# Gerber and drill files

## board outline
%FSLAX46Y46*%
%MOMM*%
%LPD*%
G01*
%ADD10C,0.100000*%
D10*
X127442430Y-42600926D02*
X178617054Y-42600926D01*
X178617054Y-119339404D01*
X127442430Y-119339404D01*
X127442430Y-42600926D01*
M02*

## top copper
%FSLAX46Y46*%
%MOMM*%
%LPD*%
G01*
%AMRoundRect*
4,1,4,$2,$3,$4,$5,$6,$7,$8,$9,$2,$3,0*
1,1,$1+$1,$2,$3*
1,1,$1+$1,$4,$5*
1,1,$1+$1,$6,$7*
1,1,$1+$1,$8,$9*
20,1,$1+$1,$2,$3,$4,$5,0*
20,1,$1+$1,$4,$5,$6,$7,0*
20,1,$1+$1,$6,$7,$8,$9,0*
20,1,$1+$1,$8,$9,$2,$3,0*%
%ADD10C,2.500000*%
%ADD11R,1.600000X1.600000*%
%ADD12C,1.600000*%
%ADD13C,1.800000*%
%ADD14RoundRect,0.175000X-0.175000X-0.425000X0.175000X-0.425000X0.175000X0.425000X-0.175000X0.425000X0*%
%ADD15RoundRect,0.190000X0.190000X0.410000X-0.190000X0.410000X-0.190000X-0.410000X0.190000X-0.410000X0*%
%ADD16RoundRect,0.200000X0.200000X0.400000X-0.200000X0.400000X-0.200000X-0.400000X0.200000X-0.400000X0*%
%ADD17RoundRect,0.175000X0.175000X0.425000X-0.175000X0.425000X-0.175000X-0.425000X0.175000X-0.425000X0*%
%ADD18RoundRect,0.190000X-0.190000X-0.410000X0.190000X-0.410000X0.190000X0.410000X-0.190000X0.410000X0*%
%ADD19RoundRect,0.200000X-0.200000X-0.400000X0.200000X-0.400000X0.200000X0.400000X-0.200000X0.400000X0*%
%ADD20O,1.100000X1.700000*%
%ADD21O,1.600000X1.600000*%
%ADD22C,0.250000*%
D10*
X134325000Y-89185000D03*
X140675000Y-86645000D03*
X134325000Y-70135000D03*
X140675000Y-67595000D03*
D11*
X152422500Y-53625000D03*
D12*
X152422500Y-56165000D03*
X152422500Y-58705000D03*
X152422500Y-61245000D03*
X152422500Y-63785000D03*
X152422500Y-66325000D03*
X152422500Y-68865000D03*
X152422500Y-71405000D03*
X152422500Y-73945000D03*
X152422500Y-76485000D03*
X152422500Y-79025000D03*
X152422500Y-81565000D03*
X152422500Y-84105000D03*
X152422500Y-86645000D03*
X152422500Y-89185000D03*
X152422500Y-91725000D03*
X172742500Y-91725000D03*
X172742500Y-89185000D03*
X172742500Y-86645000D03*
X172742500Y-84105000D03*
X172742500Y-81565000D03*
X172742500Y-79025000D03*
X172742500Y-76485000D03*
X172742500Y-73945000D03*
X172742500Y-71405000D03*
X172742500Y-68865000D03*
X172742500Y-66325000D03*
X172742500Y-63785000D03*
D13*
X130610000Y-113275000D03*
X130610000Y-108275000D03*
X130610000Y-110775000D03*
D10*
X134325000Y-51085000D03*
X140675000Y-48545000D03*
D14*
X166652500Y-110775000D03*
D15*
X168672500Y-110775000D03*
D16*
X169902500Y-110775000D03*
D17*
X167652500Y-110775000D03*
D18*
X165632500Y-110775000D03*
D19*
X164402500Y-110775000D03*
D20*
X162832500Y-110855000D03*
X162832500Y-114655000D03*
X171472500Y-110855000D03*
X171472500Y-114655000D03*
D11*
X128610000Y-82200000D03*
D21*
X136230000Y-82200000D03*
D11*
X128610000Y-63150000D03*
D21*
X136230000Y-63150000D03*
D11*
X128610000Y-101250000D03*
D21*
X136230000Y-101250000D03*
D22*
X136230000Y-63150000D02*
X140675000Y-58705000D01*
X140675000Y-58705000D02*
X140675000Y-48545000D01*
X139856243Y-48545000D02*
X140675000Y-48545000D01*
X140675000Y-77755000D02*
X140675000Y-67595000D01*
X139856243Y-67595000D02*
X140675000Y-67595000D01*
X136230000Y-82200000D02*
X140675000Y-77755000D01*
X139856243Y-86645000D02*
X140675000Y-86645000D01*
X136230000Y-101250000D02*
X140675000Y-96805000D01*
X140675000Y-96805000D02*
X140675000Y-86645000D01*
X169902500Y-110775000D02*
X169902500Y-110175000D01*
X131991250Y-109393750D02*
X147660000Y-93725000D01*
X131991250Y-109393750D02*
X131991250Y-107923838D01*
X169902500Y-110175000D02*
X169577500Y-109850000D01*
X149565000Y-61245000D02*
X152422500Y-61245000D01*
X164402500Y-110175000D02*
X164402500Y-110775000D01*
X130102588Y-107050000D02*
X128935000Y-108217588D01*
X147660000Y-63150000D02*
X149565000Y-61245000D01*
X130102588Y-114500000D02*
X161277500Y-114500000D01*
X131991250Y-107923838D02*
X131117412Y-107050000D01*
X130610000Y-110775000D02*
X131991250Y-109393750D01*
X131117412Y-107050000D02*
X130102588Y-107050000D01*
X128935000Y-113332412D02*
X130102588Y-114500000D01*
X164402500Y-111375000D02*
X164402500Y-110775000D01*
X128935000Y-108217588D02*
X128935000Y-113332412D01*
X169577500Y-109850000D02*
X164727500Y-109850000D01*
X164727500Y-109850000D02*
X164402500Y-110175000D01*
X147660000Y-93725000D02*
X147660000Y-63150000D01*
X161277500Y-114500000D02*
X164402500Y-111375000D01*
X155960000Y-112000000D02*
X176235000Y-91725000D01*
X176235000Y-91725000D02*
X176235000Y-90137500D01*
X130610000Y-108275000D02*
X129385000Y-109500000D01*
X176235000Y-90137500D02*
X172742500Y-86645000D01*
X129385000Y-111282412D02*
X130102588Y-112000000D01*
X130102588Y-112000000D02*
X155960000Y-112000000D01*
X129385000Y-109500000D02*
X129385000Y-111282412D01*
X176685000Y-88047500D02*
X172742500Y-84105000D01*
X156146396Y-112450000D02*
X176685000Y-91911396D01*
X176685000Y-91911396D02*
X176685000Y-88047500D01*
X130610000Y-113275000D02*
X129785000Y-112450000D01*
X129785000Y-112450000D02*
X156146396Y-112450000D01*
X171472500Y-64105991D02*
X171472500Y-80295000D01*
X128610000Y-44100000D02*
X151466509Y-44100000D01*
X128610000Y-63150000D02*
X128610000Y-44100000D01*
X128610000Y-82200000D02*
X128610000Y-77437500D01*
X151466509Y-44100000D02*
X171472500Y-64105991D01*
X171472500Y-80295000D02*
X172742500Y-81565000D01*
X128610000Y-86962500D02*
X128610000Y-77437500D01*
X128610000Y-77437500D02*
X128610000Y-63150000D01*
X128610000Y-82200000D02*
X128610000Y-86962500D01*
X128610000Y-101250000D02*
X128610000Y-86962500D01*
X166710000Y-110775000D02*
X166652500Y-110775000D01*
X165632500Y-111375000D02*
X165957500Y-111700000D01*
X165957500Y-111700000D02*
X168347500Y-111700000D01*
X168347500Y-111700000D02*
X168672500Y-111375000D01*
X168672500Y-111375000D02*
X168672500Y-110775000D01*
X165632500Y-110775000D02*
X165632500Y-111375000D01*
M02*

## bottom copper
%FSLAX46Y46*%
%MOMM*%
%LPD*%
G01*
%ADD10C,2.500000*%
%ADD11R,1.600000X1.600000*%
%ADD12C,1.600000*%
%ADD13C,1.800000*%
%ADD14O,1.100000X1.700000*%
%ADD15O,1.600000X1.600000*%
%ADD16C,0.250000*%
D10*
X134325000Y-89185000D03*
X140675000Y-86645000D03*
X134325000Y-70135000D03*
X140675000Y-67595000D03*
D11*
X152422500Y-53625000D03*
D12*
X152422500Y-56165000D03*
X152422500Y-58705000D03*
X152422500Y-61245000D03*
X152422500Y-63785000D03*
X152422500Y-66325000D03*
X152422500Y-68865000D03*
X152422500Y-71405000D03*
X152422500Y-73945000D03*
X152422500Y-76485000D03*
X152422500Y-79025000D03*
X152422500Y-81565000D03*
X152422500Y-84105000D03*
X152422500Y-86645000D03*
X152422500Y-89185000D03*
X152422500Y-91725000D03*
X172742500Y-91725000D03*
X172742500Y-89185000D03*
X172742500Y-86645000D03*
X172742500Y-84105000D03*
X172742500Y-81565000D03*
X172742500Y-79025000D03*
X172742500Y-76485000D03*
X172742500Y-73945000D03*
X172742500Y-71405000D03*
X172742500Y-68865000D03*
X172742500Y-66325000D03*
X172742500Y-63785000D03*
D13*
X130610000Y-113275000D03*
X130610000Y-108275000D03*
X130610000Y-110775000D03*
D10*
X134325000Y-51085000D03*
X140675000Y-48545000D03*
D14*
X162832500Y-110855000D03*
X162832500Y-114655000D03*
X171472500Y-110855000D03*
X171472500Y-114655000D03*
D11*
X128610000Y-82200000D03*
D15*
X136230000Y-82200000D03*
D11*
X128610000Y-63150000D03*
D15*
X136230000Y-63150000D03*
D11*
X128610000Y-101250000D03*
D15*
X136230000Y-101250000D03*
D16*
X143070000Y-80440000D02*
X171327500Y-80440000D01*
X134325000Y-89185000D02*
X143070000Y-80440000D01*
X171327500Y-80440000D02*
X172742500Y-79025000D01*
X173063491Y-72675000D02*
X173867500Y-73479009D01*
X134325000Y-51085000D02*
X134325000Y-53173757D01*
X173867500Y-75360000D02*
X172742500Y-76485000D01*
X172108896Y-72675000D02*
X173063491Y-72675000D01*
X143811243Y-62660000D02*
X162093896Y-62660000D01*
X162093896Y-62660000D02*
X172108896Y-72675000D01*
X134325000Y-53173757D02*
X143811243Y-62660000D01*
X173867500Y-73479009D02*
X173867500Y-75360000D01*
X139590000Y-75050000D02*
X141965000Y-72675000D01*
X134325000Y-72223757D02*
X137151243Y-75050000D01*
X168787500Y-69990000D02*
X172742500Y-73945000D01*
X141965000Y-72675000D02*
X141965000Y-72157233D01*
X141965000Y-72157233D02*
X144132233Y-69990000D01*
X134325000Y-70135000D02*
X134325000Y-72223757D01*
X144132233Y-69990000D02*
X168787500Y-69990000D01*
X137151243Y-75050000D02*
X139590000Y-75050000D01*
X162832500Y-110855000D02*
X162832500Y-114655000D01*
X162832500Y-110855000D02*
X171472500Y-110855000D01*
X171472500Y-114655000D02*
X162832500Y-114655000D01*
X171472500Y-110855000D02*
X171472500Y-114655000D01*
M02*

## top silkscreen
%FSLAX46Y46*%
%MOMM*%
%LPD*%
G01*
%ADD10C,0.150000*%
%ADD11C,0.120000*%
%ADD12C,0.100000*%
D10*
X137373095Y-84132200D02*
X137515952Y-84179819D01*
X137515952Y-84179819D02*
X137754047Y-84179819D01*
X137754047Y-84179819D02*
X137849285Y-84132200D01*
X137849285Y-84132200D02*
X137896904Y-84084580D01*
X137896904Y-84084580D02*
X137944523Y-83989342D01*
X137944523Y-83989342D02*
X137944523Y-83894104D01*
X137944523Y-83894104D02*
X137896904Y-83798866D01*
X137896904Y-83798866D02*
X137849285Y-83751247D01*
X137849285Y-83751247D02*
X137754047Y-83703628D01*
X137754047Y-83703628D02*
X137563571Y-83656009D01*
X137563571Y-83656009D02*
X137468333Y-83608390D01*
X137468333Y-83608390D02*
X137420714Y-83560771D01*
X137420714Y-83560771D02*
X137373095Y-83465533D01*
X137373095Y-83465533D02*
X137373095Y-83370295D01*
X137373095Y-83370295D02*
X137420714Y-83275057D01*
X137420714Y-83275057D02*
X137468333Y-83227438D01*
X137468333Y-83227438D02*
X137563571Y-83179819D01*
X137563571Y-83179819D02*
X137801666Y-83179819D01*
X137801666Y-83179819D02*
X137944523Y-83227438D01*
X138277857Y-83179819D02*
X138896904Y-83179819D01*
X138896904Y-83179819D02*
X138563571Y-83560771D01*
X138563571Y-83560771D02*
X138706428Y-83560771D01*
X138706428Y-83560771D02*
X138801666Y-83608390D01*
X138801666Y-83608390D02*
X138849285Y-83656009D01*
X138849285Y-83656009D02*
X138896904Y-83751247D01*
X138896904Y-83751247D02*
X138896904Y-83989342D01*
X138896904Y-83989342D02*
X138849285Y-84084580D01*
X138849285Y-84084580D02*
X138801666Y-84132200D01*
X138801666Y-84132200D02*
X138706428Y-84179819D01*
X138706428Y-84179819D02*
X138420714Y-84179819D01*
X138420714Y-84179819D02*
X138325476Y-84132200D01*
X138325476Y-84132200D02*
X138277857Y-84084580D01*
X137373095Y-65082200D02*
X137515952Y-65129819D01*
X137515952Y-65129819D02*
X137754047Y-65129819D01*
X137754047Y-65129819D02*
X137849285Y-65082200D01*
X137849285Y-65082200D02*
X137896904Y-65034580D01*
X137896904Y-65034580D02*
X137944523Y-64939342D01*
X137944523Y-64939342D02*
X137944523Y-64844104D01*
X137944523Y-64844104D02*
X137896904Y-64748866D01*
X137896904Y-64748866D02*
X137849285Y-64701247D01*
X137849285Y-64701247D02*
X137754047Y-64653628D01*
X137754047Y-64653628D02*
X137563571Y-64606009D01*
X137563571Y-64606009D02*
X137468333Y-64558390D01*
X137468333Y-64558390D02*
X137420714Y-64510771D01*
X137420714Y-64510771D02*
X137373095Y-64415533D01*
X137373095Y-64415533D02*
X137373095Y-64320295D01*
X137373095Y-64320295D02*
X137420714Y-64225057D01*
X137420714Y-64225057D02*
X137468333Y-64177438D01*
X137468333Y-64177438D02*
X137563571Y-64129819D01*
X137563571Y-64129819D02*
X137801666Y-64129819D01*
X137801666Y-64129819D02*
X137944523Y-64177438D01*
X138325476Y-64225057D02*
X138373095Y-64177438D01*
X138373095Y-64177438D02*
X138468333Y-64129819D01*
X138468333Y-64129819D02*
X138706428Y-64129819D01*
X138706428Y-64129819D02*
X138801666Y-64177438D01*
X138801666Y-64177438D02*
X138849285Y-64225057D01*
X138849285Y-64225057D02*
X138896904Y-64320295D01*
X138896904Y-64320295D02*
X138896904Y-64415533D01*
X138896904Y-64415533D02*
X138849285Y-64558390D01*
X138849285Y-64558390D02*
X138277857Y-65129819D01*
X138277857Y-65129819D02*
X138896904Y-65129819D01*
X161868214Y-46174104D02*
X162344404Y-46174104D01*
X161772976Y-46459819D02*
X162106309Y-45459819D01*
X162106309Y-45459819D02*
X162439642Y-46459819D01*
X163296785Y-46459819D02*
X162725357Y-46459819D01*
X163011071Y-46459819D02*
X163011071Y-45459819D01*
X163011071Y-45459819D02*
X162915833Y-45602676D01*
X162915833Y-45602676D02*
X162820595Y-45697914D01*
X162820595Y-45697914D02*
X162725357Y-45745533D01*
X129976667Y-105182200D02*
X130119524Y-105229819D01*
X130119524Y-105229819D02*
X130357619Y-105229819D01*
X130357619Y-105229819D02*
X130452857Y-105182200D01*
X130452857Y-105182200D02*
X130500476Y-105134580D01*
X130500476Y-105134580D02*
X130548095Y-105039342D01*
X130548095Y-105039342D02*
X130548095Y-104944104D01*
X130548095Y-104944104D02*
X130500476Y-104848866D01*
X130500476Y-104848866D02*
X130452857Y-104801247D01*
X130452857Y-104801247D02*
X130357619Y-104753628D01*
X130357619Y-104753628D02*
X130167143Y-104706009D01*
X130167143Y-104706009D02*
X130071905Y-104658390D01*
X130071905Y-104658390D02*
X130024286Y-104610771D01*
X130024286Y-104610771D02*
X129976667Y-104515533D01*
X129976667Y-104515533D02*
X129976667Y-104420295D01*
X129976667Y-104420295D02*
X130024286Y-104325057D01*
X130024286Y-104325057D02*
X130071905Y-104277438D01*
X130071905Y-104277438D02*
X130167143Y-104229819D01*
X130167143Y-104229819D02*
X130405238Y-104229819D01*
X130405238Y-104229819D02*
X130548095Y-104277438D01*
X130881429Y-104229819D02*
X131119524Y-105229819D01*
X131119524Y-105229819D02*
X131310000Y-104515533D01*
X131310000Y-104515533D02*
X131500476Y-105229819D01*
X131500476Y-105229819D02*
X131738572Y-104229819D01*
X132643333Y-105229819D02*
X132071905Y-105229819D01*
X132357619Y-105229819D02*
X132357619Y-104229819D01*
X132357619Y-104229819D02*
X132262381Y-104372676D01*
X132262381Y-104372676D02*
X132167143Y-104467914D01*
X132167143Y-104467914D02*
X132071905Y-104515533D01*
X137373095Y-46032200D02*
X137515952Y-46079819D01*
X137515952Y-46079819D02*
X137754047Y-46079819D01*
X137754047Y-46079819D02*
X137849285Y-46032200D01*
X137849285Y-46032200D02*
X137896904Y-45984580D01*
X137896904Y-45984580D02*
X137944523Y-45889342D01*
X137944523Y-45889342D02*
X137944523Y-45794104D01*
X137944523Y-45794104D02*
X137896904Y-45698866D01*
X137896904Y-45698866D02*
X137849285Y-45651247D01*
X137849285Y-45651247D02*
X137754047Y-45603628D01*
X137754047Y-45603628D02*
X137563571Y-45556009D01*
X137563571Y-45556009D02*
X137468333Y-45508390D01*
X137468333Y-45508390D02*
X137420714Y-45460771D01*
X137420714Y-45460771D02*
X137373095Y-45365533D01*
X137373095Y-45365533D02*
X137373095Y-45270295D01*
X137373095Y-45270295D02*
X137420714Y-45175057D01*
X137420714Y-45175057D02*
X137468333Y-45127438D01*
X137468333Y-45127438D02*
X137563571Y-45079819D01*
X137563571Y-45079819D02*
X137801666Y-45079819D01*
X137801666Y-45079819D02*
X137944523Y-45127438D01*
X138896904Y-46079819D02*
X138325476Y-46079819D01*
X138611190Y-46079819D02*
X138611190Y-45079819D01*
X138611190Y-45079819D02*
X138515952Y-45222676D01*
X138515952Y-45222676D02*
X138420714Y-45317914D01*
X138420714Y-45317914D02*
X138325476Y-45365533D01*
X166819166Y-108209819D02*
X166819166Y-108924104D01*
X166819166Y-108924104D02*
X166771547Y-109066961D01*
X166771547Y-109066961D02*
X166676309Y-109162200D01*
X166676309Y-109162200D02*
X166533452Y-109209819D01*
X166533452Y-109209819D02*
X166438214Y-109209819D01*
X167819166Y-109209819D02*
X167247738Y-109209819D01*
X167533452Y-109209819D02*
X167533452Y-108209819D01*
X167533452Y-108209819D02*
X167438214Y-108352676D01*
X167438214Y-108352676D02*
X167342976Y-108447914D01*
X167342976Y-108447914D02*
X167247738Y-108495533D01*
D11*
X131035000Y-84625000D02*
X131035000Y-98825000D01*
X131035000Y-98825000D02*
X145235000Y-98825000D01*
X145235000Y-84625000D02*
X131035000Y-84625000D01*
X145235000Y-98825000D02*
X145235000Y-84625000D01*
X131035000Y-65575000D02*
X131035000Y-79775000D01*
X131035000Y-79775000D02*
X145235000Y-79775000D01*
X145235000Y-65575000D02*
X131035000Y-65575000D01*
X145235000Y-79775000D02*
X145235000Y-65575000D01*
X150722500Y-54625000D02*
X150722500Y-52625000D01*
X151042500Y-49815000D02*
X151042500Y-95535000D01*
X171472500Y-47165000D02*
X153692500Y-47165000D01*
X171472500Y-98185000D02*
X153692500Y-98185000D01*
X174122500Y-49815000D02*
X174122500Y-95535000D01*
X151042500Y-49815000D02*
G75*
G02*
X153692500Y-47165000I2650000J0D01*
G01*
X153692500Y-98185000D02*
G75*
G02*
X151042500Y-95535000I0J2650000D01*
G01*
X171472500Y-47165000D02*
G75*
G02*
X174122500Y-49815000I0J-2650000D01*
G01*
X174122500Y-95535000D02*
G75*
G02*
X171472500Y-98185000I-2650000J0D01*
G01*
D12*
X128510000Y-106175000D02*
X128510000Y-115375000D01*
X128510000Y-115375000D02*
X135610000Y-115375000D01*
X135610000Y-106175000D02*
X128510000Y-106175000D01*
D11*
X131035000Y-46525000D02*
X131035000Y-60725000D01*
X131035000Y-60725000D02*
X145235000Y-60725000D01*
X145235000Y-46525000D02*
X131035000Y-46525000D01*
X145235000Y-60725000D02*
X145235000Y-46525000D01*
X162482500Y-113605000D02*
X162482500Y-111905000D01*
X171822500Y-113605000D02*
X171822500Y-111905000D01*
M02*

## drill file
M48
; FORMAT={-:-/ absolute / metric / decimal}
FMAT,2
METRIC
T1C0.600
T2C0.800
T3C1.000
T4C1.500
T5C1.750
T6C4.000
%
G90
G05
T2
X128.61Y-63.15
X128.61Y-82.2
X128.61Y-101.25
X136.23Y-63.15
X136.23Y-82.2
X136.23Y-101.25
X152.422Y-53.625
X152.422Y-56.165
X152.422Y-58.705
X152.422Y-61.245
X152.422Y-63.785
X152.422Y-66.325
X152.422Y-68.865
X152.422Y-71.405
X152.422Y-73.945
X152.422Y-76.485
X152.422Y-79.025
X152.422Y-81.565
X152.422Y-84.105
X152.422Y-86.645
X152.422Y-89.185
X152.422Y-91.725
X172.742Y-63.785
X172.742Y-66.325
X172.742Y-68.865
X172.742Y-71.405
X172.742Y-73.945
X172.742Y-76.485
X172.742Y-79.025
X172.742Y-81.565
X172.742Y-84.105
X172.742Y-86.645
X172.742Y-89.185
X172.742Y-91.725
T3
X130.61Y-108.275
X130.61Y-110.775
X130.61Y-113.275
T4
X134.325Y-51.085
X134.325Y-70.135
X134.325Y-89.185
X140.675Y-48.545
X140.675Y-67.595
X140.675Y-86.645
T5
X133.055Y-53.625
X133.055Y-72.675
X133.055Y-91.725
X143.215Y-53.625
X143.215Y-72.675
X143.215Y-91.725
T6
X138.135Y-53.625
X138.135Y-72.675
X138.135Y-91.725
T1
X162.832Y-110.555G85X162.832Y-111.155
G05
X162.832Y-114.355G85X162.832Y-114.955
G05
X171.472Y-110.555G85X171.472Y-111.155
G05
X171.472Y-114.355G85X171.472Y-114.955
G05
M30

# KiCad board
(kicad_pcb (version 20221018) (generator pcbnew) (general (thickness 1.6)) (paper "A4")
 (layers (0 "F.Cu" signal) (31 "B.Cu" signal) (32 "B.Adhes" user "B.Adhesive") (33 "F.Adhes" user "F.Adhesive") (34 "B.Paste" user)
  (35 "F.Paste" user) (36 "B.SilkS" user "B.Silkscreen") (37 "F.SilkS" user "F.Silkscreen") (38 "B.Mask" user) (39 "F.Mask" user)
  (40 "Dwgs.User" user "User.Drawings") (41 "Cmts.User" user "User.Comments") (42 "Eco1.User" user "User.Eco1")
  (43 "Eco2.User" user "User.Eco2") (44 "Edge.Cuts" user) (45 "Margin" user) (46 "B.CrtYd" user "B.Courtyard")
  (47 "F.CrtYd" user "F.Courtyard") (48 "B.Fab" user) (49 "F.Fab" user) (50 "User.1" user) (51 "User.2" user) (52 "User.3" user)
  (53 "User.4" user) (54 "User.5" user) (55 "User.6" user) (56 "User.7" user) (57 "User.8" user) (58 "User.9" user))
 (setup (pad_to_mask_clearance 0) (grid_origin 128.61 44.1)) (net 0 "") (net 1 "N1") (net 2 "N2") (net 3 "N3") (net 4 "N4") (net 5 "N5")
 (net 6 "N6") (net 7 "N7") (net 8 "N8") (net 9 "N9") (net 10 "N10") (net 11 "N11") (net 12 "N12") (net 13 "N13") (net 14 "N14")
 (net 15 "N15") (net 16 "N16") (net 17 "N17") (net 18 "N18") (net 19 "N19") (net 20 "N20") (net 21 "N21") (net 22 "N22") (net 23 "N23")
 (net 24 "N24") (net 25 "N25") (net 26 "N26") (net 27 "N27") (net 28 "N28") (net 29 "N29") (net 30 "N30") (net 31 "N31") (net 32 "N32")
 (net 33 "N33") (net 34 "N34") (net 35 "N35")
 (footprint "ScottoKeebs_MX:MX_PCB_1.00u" (layer "F.Cu") (at 138.135 91.725)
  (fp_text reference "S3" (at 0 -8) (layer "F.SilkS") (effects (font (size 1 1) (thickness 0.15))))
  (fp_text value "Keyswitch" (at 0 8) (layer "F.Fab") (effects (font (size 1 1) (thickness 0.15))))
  (fp_line (start -7.1 -7.1) (end -7.1 7.1) (stroke (width 0.12) (type solid)) (layer "F.SilkS"))
  (fp_line (start -7.1 7.1) (end 7.1 7.1) (stroke (width 0.12) (type solid)) (layer "F.SilkS"))
  (fp_line (start 7.1 -7.1) (end -7.1 -7.1) (stroke (width 0.12) (type solid)) (layer "F.SilkS"))
  (fp_line (start 7.1 7.1) (end 7.1 -7.1) (stroke (width 0.12) (type solid)) (layer "F.SilkS"))
  (pad "" np_thru_hole circle (at -5.08 0) (size 1.75 1.75) (drill 1.75) (layers "*.Cu" "*.Mask"))
  (pad "" np_thru_hole circle (at 0 0) (size 4 4) (drill 4) (layers "*.Cu" "*.Mask"))
  (pad "" np_thru_hole circle (at 5.08 0) (size 1.75 1.75) (drill 1.75) (layers "*.Cu" "*.Mask"))
  (pad "1" thru_hole circle (at -3.81 -2.54) (size 2.5 2.5) (drill 1.5) (layers "*.Cu" "*.Mask") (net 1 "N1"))
  (pad "2" thru_hole circle (at 2.54 -5.08) (size 2.5 2.5) (drill 1.5) (layers "*.Cu" "*.Mask") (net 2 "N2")))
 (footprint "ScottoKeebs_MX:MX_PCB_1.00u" (layer "F.Cu") (at 138.135 72.675)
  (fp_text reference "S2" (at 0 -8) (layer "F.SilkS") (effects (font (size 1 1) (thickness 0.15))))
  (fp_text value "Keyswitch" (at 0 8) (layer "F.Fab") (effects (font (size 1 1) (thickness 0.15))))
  (fp_line (start -7.1 -7.1) (end -7.1 7.1) (stroke (width 0.12) (type solid)) (layer "F.SilkS"))
  (fp_line (start -7.1 7.1) (end 7.1 7.1) (stroke (width 0.12) (type solid)) (layer "F.SilkS"))
  (fp_line (start 7.1 -7.1) (end -7.1 -7.1) (stroke (width 0.12) (type solid)) (layer "F.SilkS"))
  (fp_line (start 7.1 7.1) (end 7.1 -7.1) (stroke (width 0.12) (type solid)) (layer "F.SilkS"))
  (pad "" np_thru_hole circle (at -5.08 0) (size 1.75 1.75) (drill 1.75) (layers "*.Cu" "*.Mask"))
  (pad "" np_thru_hole circle (at 0 0) (size 4 4) (drill 4) (layers "*.Cu" "*.Mask"))
  (pad "" np_thru_hole circle (at 5.08 0) (size 1.75 1.75) (drill 1.75) (layers "*.Cu" "*.Mask"))
  (pad "1" thru_hole circle (at -3.81 -2.54) (size 2.5 2.5) (drill 1.5) (layers "*.Cu" "*.Mask") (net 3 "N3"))
  (pad "2" thru_hole circle (at 2.54 -5.08) (size 2.5 2.5) (drill 1.5) (layers "*.Cu" "*.Mask") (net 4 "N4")))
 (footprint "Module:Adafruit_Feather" (layer "F.Cu") (at 152.4225 53.625)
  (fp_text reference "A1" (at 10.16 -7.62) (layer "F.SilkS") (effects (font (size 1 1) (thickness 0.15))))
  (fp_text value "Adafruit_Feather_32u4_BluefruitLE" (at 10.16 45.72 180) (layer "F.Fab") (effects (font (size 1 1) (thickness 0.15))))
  (fp_line (start -1.7 1) (end -1.7 -1) (stroke (width 0.12) (type solid)) (layer "F.SilkS"))
  (fp_line (start -1.38 -3.81) (end -1.38 41.91) (stroke (width 0.12) (type solid)) (layer "F.SilkS"))
  (fp_line (start 19.05 -6.46) (end 1.27 -6.46) (stroke (width 0.12) (type solid)) (layer "F.SilkS"))
  (fp_line (start 19.05 44.56) (end 1.27 44.56) (stroke (width 0.12) (type solid)) (layer "F.SilkS"))
  (fp_line (start 21.7 -3.81) (end 21.7 41.91) (stroke (width 0.12) (type solid)) (layer "F.SilkS"))
  (fp_arc (start -1.38 -3.81) (mid -0.603833 -5.683833) (end 1.27 -6.46) (stroke (width 0.12) (type solid)) (layer "F.SilkS"))
  (fp_arc (start 1.27 44.56) (mid -0.603833 43.783833) (end -1.38 41.91) (stroke (width 0.12) (type solid)) (layer "F.SilkS"))
  (fp_arc (start 19.05 -6.46) (mid 20.923833 -5.683833) (end 21.7 -3.81) (stroke (width 0.12) (type solid)) (layer "F.SilkS"))
  (fp_arc (start 21.7 41.91) (mid 20.923833 43.783833) (end 19.05 44.56) (stroke (width 0.12) (type solid)) (layer "F.SilkS"))
  (pad "1" thru_hole rect (at 0 0 180) (size 1.6 1.6) (drill 0.8) (layers "*.Cu" "*.Mask") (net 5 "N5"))
  (pad "2" thru_hole circle (at 0 2.54 180) (size 1.6 1.6) (drill 0.8) (layers "*.Cu" "*.Mask") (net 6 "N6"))
  (pad "3" thru_hole circle (at 0 5.08 180) (size 1.6 1.6) (drill 0.8) (layers "*.Cu" "*.Mask") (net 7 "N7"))
  (pad "4" thru_hole circle (at 0 7.62 180) (size 1.6 1.6) (drill 0.8) (layers "*.Cu" "*.Mask") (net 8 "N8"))
  (pad "5" thru_hole circle (at 0 10.16 180) (size 1.6 1.6) (drill 0.8) (layers "*.Cu" "*.Mask") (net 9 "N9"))
  (pad "6" thru_hole circle (at 0 12.7 180) (size 1.6 1.6) (drill 0.8) (layers "*.Cu" "*.Mask") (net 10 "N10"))
  (pad "7" thru_hole circle (at 0 15.24 180) (size 1.6 1.6) (drill 0.8) (layers "*.Cu" "*.Mask") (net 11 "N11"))
  (pad "8" thru_hole circle (at 0 17.78 180) (size 1.6 1.6) (drill 0.8) (layers "*.Cu" "*.Mask") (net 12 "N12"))
  (pad "9" thru_hole circle (at 0 20.32 180) (size 1.6 1.6) (drill 0.8) (layers "*.Cu" "*.Mask") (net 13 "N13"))
  (pad "10" thru_hole circle (at 0 22.86 180) (size 1.6 1.6) (drill 0.8) (layers "*.Cu" "*.Mask") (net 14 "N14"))
  (pad "11" thru_hole circle (at 0 25.4 180) (size 1.6 1.6) (drill 0.8) (layers "*.Cu" "*.Mask") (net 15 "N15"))
  (pad "12" thru_hole circle (at 0 27.94 180) (size 1.6 1.6) (drill 0.8) (layers "*.Cu" "*.Mask") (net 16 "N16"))
  (pad "13" thru_hole circle (at 0 30.48 180) (size 1.6 1.6) (drill 0.8) (layers "*.Cu" "*.Mask") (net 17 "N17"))
  (pad "14" thru_hole circle (at 0 33.02 180) (size 1.6 1.6) (drill 0.8) (layers "*.Cu" "*.Mask") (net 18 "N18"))
  (pad "15" thru_hole circle (at 0 35.56 180) (size 1.6 1.6) (drill 0.8) (layers "*.Cu" "*.Mask") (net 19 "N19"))
  (pad "16" thru_hole circle (at 0 38.1 180) (size 1.6 1.6) (drill 0.8) (layers "*.Cu" "*.Mask") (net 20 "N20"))
  (pad "17" thru_hole circle (at 20.32 38.1 180) (size 1.6 1.6) (drill 0.8) (layers "*.Cu" "*.Mask") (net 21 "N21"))
  (pad "18" thru_hole circle (at 20.32 35.56 180) (size 1.6 1.6) (drill 0.8) (layers "*.Cu" "*.Mask") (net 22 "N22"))
  (pad "19" thru_hole circle (at 20.32 33.02 180) (size 1.6 1.6) (drill 0.8) (layers "*.Cu" "*.Mask") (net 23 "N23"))
  (pad "20" thru_hole circle (at 20.32 30.48 180) (size 1.6 1.6) (drill 0.8) (layers "*.Cu" "*.Mask") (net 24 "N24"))
  (pad "21" thru_hole circle (at 20.32 27.94 180) (size 1.6 1.6) (drill 0.8) (layers "*.Cu" "*.Mask") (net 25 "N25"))
  (pad "22" thru_hole circle (at 20.32 25.4 180) (size 1.6 1.6) (drill 0.8) (layers "*.Cu" "*.Mask") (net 1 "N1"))
  (pad "23" thru_hole circle (at 20.32 22.86 180) (size 1.6 1.6) (drill 0.8) (layers "*.Cu" "*.Mask") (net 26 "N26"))
  (pad "24" thru_hole circle (at 20.32 20.32 180) (size 1.6 1.6) (drill 0.8) (layers "*.Cu" "*.Mask") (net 3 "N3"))
  (pad "25" thru_hole circle (at 20.32 17.78 180) (size 1.6 1.6) (drill 0.8) (layers "*.Cu" "*.Mask") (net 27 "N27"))
  (pad "26" thru_hole circle (at 20.32 15.24 180) (size 1.6 1.6) (drill 0.8) (layers "*.Cu" "*.Mask") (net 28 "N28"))
  (pad "27" thru_hole circle (at 20.32 12.7 180) (size 1.6 1.6) (drill 0.8) (layers "*.Cu" "*.Mask") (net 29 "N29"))
  (pad "28" thru_hole circle (at 20.32 10.16 180) (size 1.6 1.6) (drill 0.8) (layers "*.Cu" "*.Mask") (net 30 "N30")))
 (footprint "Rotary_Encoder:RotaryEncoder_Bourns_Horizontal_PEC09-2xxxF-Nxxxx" (layer "F.Cu") (at 130.61 113.275)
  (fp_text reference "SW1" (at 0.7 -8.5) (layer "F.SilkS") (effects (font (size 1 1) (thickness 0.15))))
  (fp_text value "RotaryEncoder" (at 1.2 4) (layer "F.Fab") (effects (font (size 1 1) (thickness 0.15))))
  (fp_line (start -2.1 -7.1) (end -2.1 2.1) (stroke (width 0.1) (type solid)) (layer "F.SilkS"))
  (fp_line (start -2.1 2.1) (end 5 2.1) (stroke (width 0.1) (type solid)) (layer "F.SilkS"))
  (fp_line (start 5 -7.1) (end -2.1 -7.1) (stroke (width 0.1) (type solid)) (layer "F.SilkS"))
  (pad "A" thru_hole circle (at 0 0) (size 1.8 1.8) (drill 1) (layers "*.Cu" "*.Mask") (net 24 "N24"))
  (pad "B" thru_hole circle (at 0 -5) (size 1.8 1.8) (drill 1) (layers "*.Cu" "*.Mask") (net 23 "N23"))
  (pad "C" thru_hole circle (at 0 -2.5) (size 1.8 1.8) (drill 1) (layers "*.Cu" "*.Mask") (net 8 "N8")))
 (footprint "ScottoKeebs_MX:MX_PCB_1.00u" (layer "F.Cu") (at 138.135 53.625)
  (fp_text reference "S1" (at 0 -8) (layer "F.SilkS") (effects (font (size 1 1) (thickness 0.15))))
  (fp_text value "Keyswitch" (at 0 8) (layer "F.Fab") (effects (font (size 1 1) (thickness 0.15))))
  (fp_line (start -7.1 -7.1) (end -7.1 7.1) (stroke (width 0.12) (type solid)) (layer "F.SilkS"))
  (fp_line (start -7.1 7.1) (end 7.1 7.1) (stroke (width 0.12) (type solid)) (layer "F.SilkS"))
  (fp_line (start 7.1 -7.1) (end -7.1 -7.1) (stroke (width 0.12) (type solid)) (layer "F.SilkS"))
  (fp_line (start 7.1 7.1) (end 7.1 -7.1) (stroke (width 0.12) (type solid)) (layer "F.SilkS"))
  (pad "" np_thru_hole circle (at -5.08 0) (size 1.75 1.75) (drill 1.75) (layers "*.Cu" "*.Mask"))
  (pad "" np_thru_hole circle (at 0 0) (size 4 4) (drill 4) (layers "*.Cu" "*.Mask"))
  (pad "" np_thru_hole circle (at 5.08 0) (size 1.75 1.75) (drill 1.75) (layers "*.Cu" "*.Mask"))
  (pad "1" thru_hole circle (at -3.81 -2.54) (size 2.5 2.5) (drill 1.5) (layers "*.Cu" "*.Mask") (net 26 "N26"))
  (pad "2" thru_hole circle (at 2.54 -5.08) (size 2.5 2.5) (drill 1.5) (layers "*.Cu" "*.Mask") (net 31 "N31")))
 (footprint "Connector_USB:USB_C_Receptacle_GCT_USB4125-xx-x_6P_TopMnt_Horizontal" (layer "F.Cu") (at 167.1525 113.855)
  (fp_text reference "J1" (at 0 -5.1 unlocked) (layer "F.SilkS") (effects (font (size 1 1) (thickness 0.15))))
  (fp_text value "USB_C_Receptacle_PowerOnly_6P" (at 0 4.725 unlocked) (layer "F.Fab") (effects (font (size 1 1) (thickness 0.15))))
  (fp_line (start -4.67 -0.25) (end -4.67 -1.95) (stroke (width 0.12) (type solid)) (layer "F.SilkS"))
  (fp_line (start 4.67 -0.25) (end 4.67 -1.95) (stroke (width 0.12) (type solid)) (layer "F.SilkS"))
  (pad "A5" smd roundrect (at -0.5 -3.08) (size 0.7 1.2) (layers "F.Cu" "F.Paste" "F.Mask") (roundrect_rratio 0.25) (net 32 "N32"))
  (pad "A9" smd roundrect (at 1.52 -3.08 180) (size 0.76 1.2) (layers "F.Cu" "F.Paste" "F.Mask") (roundrect_rratio 0.25) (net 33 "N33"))
  (pad "A12" smd roundrect (at 2.75 -3.08 180) (size 0.8 1.2) (layers "F.Cu" "F.Paste" "F.Mask") (roundrect_rratio 0.25) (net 8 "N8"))
  (pad "B5" smd roundrect (at 0.5 -3.08 180) (size 0.7 1.2) (layers "F.Cu" "F.Paste" "F.Mask") (roundrect_rratio 0.25) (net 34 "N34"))
  (pad "B9" smd roundrect (at -1.52 -3.08) (size 0.76 1.2) (layers "F.Cu" "F.Paste" "F.Mask") (roundrect_rratio 0.25) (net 33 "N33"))
  (pad "B12" smd roundrect (at -2.75 -3.08) (size 0.8 1.2) (layers "F.Cu" "F.Paste" "F.Mask") (roundrect_rratio 0.25) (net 8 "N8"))
  (pad "S1" thru_hole oval (at -4.32 -3) (size 1.1 1.7) (drill oval 0.6 1.2) (layers "*.Cu" "*.Mask" "F.Paste") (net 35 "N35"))
  (pad "S1" thru_hole oval (at -4.32 0.8) (size 1.1 1.7) (drill oval 0.6 1.2) (layers "*.Cu" "*.Mask" "F.Paste") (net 35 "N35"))
  (pad "S1" thru_hole oval (at 4.32 -3) (size 1.1 1.7) (drill oval 0.6 1.2) (layers "*.Cu" "*.Mask" "F.Paste") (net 35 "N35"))
  (pad "S1" thru_hole oval (at 4.32 0.8) (size 1.1 1.7) (drill oval 0.6 1.2) (layers "*.Cu" "*.Mask" "F.Paste") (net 35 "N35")))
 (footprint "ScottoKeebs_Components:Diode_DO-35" (layer "B.Cu") (at 128.61 82.2)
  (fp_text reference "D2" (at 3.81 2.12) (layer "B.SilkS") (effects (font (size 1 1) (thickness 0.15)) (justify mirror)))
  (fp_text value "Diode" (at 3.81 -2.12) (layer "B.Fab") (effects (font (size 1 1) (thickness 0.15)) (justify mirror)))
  (pad "1" thru_hole rect (at 0 0) (size 1.6 1.6) (drill 0.8) (layers "*.Cu" "*.Mask") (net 25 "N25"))
  (pad "2" thru_hole oval (at 7.62 0) (size 1.6 1.6) (drill 0.8) (layers "*.Cu" "*.Mask") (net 4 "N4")))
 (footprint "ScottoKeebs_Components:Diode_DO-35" (layer "B.Cu") (at 128.61 63.15)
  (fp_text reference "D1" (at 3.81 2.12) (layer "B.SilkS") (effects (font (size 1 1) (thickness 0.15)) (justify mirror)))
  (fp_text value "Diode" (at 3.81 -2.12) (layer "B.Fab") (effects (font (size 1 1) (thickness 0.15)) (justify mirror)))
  (pad "1" thru_hole rect (at 0 0) (size 1.6 1.6) (drill 0.8) (layers "*.Cu" "*.Mask") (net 25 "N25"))
  (pad "2" thru_hole oval (at 7.62 0) (size 1.6 1.6) (drill 0.8) (layers "*.Cu" "*.Mask") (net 31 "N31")))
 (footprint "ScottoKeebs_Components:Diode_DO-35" (layer "B.Cu") (at 128.61 101.25)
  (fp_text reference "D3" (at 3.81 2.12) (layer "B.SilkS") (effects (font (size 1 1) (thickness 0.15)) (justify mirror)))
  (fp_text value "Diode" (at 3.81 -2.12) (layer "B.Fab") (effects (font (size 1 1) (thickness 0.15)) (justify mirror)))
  (pad "1" thru_hole rect (at 0 0) (size 1.6 1.6) (drill 0.8) (layers "*.Cu" "*.Mask") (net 25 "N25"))
  (pad "2" thru_hole oval (at 7.62 0) (size 1.6 1.6) (drill 0.8) (layers "*.Cu" "*.Mask") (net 2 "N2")))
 (gr_rect (start 127.44243 42.600926) (end 178.617054 119.339404) (stroke (width 0.1) (type default)) (fill none) (layer "Edge.Cuts"))
 (segment (start 136.23 63.15) (end 140.675 58.705) (width 0.25) (layer "F.Cu") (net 31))
 (segment (start 140.675 58.705) (end 140.675 48.545) (width 0.25) (layer "F.Cu") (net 31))
 (segment (start 139.856243 48.545) (end 140.675 48.545) (width 0.25) (layer "F.Cu") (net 31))
 (segment (start 140.675 77.755) (end 140.675 67.595) (width 0.25) (layer "F.Cu") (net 4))
 (segment (start 139.856243 67.595) (end 140.675 67.595) (width 0.25) (layer "F.Cu") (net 4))
 (segment (start 136.23 82.2) (end 140.675 77.755) (width 0.25) (layer "F.Cu") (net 4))
 (segment (start 139.856243 86.645) (end 140.675 86.645) (width 0.25) (layer "F.Cu") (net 2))
 (segment (start 136.23 101.25) (end 140.675 96.805) (width 0.25) (layer "F.Cu") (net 2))
 (segment (start 140.675 96.805) (end 140.675 86.645) (width 0.25) (layer "F.Cu") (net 2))
 (segment (start 169.9025 110.775) (end 169.9025 110.175) (width 0.25) (layer "F.Cu") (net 8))
 (segment (start 131.99125 109.39375) (end 147.66 93.725) (width 0.25) (layer "F.Cu") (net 8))
 (segment (start 131.99125 109.39375) (end 131.99125 107.923838) (width 0.25) (layer "F.Cu") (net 8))
 (segment (start 169.9025 110.175) (end 169.5775 109.85) (width 0.25) (layer "F.Cu") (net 8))
 (segment (start 149.565 61.245) (end 152.4225 61.245) (width 0.25) (layer "F.Cu") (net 8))
 (segment (start 164.4025 110.175) (end 164.4025 110.775) (width 0.25) (layer "F.Cu") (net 8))
 (segment (start 130.102588 107.05) (end 128.935 108.217588) (width 0.25) (layer "F.Cu") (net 8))
 (segment (start 147.66 63.15) (end 149.565 61.245) (width 0.25) (layer "F.Cu") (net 8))
 (segment (start 130.102588 114.5) (end 161.2775 114.5) (width 0.25) (layer "F.Cu") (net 8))
 (segment (start 131.99125 107.923838) (end 131.117412 107.05) (width 0.25) (layer "F.Cu") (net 8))
 (segment (start 130.61 110.775) (end 131.99125 109.39375) (width 0.25) (layer "F.Cu") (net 8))
 (segment (start 131.117412 107.05) (end 130.102588 107.05) (width 0.25) (layer "F.Cu") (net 8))
 (segment (start 128.935 113.332412) (end 130.102588 114.5) (width 0.25) (layer "F.Cu") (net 8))
 (segment (start 164.4025 111.375) (end 164.4025 110.775) (width 0.25) (layer "F.Cu") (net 8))
 (segment (start 128.935 108.217588) (end 128.935 113.332412) (width 0.25) (layer "F.Cu") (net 8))
 (segment (start 169.5775 109.85) (end 164.7275 109.85) (width 0.25) (layer "F.Cu") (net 8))
 (segment (start 164.7275 109.85) (end 164.4025 110.175) (width 0.25) (layer "F.Cu") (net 8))
 (segment (start 147.66 93.725) (end 147.66 63.15) (width 0.25) (layer "F.Cu") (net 8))
 (segment (start 161.2775 114.5) (end 164.4025 111.375) (width 0.25) (layer "F.Cu") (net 8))
 (segment (start 155.96 112) (end 176.235 91.725) (width 0.25) (layer "F.Cu") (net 23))
 (segment (start 176.235 91.725) (end 176.235 90.1375) (width 0.25) (layer "F.Cu") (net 23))
 (segment (start 130.61 108.275) (end 129.385 109.5) (width 0.25) (layer "F.Cu") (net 23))
 (segment (start 176.235 90.1375) (end 172.7425 86.645) (width 0.25) (layer "F.Cu") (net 23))
 (segment (start 129.385 111.282412) (end 130.102588 112) (width 0.25) (layer "F.Cu") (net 23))
 (segment (start 130.102588 112) (end 155.96 112) (width 0.25) (layer "F.Cu") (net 23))
 (segment (start 129.385 109.5) (end 129.385 111.282412) (width 0.25) (layer "F.Cu") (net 23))
 (segment (start 176.685 88.0475) (end 172.7425 84.105) (width 0.25) (layer "F.Cu") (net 24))
 (segment (start 156.146396 112.45) (end 176.685 91.911396) (width 0.25) (layer "F.Cu") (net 24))
 (segment (start 176.685 91.911396) (end 176.685 88.0475) (width 0.25) (layer "F.Cu") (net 24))
 (segment (start 130.61 113.275) (end 129.785 112.45) (width 0.25) (layer "F.Cu") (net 24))
 (segment (start 129.785 112.45) (end 156.146396 112.45) (width 0.25) (layer "F.Cu") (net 24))
 (segment (start 171.4725 64.105991) (end 171.4725 80.295) (width 0.25) (layer "F.Cu") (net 25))
 (segment (start 128.61 44.1) (end 151.466509 44.1) (width 0.25) (layer "F.Cu") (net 25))
 (segment (start 128.61 63.15) (end 128.61 44.1) (width 0.25) (layer "F.Cu") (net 25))
 (segment (start 128.61 82.2) (end 128.61 77.4375) (width 0.25) (layer "F.Cu") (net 25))
 (segment (start 151.466509 44.1) (end 171.4725 64.105991) (width 0.25) (layer "F.Cu") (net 25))
 (segment (start 171.4725 80.295) (end 172.7425 81.565) (width 0.25) (layer "F.Cu") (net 25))
 (segment (start 128.61 86.9625) (end 128.61 77.4375) (width 0.25) (layer "F.Cu") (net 25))
 (segment (start 128.61 77.4375) (end 128.61 63.15) (width 0.25) (layer "F.Cu") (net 25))
 (segment (start 128.61 82.2) (end 128.61 86.9625) (width 0.25) (layer "F.Cu") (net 25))
 (segment (start 128.61 101.25) (end 128.61 86.9625) (width 0.25) (layer "F.Cu") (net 25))
 (segment (start 143.07 80.44) (end 171.3275 80.44) (width 0.25) (layer "B.Cu") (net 1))
 (segment (start 134.325 89.185) (end 143.07 80.44) (width 0.25) (layer "B.Cu") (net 1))
 (segment (start 171.3275 80.44) (end 172.7425 79.025) (width 0.25) (layer "B.Cu") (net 1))
 (segment (start 173.063491 72.675) (end 173.8675 73.479009) (width 0.25) (layer "B.Cu") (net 26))
 (segment (start 134.325 51.085) (end 134.325 53.173757) (width 0.25) (layer "B.Cu") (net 26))
 (segment (start 173.8675 75.36) (end 172.7425 76.485) (width 0.25) (layer "B.Cu") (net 26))
 (segment (start 172.108896 72.675) (end 173.063491 72.675) (width 0.25) (layer "B.Cu") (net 26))
 (segment (start 143.811243 62.66) (end 162.093896 62.66) (width 0.25) (layer "B.Cu") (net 26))
 (segment (start 162.093896 62.66) (end 172.108896 72.675) (width 0.25) (layer "B.Cu") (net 26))
 (segment (start 134.325 53.173757) (end 143.811243 62.66) (width 0.25) (layer "B.Cu") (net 26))
 (segment (start 173.8675 73.479009) (end 173.8675 75.36) (width 0.25) (layer "B.Cu") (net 26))
 (segment (start 139.59 75.05) (end 141.965 72.675) (width 0.25) (layer "B.Cu") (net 3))
 (segment (start 134.325 72.223757) (end 137.151243 75.05) (width 0.25) (layer "B.Cu") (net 3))
 (segment (start 168.7875 69.99) (end 172.7425 73.945) (width 0.25) (layer "B.Cu") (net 3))
 (segment (start 141.965 72.675) (end 141.965 72.157233) (width 0.25) (layer "B.Cu") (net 3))
 (segment (start 141.965 72.157233) (end 144.132233 69.99) (width 0.25) (layer "B.Cu") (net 3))
 (segment (start 134.325 70.135) (end 134.325 72.223757) (width 0.25) (layer "B.Cu") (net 3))
 (segment (start 144.132233 69.99) (end 168.7875 69.99) (width 0.25) (layer "B.Cu") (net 3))
 (segment (start 137.151243 75.05) (end 139.59 75.05) (width 0.25) (layer "B.Cu") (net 3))
 (segment (start 166.71 110.775) (end 166.6525 110.775) (width 0.25) (layer "F.Cu") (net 32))
 (segment (start 165.6325 111.375) (end 165.9575 111.7) (width 0.25) (layer "F.Cu") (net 33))
 (segment (start 165.9575 111.7) (end 168.3475 111.7) (width 0.25) (layer "F.Cu") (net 33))
 (segment (start 168.3475 111.7) (end 168.6725 111.375) (width 0.25) (layer "F.Cu") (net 33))
 (segment (start 168.6725 111.375) (end 168.6725 110.775) (width 0.25) (layer "F.Cu") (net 33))
 (segment (start 165.6325 110.775) (end 165.6325 111.375) (width 0.25) (layer "F.Cu") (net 33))
 (segment (start 162.8325 110.855) (end 162.8325 114.655) (width 0.25) (layer "B.Cu") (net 35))
 (segment (start 162.8325 110.855) (end 171.4725 110.855) (width 0.25) (layer "B.Cu") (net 35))
 (segment (start 171.4725 114.655) (end 162.8325 114.655) (width 0.25) (layer "B.Cu") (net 35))
 (segment (start 171.4725 110.855) (end 171.4725 114.655) (width 0.25) (layer "B.Cu") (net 35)))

